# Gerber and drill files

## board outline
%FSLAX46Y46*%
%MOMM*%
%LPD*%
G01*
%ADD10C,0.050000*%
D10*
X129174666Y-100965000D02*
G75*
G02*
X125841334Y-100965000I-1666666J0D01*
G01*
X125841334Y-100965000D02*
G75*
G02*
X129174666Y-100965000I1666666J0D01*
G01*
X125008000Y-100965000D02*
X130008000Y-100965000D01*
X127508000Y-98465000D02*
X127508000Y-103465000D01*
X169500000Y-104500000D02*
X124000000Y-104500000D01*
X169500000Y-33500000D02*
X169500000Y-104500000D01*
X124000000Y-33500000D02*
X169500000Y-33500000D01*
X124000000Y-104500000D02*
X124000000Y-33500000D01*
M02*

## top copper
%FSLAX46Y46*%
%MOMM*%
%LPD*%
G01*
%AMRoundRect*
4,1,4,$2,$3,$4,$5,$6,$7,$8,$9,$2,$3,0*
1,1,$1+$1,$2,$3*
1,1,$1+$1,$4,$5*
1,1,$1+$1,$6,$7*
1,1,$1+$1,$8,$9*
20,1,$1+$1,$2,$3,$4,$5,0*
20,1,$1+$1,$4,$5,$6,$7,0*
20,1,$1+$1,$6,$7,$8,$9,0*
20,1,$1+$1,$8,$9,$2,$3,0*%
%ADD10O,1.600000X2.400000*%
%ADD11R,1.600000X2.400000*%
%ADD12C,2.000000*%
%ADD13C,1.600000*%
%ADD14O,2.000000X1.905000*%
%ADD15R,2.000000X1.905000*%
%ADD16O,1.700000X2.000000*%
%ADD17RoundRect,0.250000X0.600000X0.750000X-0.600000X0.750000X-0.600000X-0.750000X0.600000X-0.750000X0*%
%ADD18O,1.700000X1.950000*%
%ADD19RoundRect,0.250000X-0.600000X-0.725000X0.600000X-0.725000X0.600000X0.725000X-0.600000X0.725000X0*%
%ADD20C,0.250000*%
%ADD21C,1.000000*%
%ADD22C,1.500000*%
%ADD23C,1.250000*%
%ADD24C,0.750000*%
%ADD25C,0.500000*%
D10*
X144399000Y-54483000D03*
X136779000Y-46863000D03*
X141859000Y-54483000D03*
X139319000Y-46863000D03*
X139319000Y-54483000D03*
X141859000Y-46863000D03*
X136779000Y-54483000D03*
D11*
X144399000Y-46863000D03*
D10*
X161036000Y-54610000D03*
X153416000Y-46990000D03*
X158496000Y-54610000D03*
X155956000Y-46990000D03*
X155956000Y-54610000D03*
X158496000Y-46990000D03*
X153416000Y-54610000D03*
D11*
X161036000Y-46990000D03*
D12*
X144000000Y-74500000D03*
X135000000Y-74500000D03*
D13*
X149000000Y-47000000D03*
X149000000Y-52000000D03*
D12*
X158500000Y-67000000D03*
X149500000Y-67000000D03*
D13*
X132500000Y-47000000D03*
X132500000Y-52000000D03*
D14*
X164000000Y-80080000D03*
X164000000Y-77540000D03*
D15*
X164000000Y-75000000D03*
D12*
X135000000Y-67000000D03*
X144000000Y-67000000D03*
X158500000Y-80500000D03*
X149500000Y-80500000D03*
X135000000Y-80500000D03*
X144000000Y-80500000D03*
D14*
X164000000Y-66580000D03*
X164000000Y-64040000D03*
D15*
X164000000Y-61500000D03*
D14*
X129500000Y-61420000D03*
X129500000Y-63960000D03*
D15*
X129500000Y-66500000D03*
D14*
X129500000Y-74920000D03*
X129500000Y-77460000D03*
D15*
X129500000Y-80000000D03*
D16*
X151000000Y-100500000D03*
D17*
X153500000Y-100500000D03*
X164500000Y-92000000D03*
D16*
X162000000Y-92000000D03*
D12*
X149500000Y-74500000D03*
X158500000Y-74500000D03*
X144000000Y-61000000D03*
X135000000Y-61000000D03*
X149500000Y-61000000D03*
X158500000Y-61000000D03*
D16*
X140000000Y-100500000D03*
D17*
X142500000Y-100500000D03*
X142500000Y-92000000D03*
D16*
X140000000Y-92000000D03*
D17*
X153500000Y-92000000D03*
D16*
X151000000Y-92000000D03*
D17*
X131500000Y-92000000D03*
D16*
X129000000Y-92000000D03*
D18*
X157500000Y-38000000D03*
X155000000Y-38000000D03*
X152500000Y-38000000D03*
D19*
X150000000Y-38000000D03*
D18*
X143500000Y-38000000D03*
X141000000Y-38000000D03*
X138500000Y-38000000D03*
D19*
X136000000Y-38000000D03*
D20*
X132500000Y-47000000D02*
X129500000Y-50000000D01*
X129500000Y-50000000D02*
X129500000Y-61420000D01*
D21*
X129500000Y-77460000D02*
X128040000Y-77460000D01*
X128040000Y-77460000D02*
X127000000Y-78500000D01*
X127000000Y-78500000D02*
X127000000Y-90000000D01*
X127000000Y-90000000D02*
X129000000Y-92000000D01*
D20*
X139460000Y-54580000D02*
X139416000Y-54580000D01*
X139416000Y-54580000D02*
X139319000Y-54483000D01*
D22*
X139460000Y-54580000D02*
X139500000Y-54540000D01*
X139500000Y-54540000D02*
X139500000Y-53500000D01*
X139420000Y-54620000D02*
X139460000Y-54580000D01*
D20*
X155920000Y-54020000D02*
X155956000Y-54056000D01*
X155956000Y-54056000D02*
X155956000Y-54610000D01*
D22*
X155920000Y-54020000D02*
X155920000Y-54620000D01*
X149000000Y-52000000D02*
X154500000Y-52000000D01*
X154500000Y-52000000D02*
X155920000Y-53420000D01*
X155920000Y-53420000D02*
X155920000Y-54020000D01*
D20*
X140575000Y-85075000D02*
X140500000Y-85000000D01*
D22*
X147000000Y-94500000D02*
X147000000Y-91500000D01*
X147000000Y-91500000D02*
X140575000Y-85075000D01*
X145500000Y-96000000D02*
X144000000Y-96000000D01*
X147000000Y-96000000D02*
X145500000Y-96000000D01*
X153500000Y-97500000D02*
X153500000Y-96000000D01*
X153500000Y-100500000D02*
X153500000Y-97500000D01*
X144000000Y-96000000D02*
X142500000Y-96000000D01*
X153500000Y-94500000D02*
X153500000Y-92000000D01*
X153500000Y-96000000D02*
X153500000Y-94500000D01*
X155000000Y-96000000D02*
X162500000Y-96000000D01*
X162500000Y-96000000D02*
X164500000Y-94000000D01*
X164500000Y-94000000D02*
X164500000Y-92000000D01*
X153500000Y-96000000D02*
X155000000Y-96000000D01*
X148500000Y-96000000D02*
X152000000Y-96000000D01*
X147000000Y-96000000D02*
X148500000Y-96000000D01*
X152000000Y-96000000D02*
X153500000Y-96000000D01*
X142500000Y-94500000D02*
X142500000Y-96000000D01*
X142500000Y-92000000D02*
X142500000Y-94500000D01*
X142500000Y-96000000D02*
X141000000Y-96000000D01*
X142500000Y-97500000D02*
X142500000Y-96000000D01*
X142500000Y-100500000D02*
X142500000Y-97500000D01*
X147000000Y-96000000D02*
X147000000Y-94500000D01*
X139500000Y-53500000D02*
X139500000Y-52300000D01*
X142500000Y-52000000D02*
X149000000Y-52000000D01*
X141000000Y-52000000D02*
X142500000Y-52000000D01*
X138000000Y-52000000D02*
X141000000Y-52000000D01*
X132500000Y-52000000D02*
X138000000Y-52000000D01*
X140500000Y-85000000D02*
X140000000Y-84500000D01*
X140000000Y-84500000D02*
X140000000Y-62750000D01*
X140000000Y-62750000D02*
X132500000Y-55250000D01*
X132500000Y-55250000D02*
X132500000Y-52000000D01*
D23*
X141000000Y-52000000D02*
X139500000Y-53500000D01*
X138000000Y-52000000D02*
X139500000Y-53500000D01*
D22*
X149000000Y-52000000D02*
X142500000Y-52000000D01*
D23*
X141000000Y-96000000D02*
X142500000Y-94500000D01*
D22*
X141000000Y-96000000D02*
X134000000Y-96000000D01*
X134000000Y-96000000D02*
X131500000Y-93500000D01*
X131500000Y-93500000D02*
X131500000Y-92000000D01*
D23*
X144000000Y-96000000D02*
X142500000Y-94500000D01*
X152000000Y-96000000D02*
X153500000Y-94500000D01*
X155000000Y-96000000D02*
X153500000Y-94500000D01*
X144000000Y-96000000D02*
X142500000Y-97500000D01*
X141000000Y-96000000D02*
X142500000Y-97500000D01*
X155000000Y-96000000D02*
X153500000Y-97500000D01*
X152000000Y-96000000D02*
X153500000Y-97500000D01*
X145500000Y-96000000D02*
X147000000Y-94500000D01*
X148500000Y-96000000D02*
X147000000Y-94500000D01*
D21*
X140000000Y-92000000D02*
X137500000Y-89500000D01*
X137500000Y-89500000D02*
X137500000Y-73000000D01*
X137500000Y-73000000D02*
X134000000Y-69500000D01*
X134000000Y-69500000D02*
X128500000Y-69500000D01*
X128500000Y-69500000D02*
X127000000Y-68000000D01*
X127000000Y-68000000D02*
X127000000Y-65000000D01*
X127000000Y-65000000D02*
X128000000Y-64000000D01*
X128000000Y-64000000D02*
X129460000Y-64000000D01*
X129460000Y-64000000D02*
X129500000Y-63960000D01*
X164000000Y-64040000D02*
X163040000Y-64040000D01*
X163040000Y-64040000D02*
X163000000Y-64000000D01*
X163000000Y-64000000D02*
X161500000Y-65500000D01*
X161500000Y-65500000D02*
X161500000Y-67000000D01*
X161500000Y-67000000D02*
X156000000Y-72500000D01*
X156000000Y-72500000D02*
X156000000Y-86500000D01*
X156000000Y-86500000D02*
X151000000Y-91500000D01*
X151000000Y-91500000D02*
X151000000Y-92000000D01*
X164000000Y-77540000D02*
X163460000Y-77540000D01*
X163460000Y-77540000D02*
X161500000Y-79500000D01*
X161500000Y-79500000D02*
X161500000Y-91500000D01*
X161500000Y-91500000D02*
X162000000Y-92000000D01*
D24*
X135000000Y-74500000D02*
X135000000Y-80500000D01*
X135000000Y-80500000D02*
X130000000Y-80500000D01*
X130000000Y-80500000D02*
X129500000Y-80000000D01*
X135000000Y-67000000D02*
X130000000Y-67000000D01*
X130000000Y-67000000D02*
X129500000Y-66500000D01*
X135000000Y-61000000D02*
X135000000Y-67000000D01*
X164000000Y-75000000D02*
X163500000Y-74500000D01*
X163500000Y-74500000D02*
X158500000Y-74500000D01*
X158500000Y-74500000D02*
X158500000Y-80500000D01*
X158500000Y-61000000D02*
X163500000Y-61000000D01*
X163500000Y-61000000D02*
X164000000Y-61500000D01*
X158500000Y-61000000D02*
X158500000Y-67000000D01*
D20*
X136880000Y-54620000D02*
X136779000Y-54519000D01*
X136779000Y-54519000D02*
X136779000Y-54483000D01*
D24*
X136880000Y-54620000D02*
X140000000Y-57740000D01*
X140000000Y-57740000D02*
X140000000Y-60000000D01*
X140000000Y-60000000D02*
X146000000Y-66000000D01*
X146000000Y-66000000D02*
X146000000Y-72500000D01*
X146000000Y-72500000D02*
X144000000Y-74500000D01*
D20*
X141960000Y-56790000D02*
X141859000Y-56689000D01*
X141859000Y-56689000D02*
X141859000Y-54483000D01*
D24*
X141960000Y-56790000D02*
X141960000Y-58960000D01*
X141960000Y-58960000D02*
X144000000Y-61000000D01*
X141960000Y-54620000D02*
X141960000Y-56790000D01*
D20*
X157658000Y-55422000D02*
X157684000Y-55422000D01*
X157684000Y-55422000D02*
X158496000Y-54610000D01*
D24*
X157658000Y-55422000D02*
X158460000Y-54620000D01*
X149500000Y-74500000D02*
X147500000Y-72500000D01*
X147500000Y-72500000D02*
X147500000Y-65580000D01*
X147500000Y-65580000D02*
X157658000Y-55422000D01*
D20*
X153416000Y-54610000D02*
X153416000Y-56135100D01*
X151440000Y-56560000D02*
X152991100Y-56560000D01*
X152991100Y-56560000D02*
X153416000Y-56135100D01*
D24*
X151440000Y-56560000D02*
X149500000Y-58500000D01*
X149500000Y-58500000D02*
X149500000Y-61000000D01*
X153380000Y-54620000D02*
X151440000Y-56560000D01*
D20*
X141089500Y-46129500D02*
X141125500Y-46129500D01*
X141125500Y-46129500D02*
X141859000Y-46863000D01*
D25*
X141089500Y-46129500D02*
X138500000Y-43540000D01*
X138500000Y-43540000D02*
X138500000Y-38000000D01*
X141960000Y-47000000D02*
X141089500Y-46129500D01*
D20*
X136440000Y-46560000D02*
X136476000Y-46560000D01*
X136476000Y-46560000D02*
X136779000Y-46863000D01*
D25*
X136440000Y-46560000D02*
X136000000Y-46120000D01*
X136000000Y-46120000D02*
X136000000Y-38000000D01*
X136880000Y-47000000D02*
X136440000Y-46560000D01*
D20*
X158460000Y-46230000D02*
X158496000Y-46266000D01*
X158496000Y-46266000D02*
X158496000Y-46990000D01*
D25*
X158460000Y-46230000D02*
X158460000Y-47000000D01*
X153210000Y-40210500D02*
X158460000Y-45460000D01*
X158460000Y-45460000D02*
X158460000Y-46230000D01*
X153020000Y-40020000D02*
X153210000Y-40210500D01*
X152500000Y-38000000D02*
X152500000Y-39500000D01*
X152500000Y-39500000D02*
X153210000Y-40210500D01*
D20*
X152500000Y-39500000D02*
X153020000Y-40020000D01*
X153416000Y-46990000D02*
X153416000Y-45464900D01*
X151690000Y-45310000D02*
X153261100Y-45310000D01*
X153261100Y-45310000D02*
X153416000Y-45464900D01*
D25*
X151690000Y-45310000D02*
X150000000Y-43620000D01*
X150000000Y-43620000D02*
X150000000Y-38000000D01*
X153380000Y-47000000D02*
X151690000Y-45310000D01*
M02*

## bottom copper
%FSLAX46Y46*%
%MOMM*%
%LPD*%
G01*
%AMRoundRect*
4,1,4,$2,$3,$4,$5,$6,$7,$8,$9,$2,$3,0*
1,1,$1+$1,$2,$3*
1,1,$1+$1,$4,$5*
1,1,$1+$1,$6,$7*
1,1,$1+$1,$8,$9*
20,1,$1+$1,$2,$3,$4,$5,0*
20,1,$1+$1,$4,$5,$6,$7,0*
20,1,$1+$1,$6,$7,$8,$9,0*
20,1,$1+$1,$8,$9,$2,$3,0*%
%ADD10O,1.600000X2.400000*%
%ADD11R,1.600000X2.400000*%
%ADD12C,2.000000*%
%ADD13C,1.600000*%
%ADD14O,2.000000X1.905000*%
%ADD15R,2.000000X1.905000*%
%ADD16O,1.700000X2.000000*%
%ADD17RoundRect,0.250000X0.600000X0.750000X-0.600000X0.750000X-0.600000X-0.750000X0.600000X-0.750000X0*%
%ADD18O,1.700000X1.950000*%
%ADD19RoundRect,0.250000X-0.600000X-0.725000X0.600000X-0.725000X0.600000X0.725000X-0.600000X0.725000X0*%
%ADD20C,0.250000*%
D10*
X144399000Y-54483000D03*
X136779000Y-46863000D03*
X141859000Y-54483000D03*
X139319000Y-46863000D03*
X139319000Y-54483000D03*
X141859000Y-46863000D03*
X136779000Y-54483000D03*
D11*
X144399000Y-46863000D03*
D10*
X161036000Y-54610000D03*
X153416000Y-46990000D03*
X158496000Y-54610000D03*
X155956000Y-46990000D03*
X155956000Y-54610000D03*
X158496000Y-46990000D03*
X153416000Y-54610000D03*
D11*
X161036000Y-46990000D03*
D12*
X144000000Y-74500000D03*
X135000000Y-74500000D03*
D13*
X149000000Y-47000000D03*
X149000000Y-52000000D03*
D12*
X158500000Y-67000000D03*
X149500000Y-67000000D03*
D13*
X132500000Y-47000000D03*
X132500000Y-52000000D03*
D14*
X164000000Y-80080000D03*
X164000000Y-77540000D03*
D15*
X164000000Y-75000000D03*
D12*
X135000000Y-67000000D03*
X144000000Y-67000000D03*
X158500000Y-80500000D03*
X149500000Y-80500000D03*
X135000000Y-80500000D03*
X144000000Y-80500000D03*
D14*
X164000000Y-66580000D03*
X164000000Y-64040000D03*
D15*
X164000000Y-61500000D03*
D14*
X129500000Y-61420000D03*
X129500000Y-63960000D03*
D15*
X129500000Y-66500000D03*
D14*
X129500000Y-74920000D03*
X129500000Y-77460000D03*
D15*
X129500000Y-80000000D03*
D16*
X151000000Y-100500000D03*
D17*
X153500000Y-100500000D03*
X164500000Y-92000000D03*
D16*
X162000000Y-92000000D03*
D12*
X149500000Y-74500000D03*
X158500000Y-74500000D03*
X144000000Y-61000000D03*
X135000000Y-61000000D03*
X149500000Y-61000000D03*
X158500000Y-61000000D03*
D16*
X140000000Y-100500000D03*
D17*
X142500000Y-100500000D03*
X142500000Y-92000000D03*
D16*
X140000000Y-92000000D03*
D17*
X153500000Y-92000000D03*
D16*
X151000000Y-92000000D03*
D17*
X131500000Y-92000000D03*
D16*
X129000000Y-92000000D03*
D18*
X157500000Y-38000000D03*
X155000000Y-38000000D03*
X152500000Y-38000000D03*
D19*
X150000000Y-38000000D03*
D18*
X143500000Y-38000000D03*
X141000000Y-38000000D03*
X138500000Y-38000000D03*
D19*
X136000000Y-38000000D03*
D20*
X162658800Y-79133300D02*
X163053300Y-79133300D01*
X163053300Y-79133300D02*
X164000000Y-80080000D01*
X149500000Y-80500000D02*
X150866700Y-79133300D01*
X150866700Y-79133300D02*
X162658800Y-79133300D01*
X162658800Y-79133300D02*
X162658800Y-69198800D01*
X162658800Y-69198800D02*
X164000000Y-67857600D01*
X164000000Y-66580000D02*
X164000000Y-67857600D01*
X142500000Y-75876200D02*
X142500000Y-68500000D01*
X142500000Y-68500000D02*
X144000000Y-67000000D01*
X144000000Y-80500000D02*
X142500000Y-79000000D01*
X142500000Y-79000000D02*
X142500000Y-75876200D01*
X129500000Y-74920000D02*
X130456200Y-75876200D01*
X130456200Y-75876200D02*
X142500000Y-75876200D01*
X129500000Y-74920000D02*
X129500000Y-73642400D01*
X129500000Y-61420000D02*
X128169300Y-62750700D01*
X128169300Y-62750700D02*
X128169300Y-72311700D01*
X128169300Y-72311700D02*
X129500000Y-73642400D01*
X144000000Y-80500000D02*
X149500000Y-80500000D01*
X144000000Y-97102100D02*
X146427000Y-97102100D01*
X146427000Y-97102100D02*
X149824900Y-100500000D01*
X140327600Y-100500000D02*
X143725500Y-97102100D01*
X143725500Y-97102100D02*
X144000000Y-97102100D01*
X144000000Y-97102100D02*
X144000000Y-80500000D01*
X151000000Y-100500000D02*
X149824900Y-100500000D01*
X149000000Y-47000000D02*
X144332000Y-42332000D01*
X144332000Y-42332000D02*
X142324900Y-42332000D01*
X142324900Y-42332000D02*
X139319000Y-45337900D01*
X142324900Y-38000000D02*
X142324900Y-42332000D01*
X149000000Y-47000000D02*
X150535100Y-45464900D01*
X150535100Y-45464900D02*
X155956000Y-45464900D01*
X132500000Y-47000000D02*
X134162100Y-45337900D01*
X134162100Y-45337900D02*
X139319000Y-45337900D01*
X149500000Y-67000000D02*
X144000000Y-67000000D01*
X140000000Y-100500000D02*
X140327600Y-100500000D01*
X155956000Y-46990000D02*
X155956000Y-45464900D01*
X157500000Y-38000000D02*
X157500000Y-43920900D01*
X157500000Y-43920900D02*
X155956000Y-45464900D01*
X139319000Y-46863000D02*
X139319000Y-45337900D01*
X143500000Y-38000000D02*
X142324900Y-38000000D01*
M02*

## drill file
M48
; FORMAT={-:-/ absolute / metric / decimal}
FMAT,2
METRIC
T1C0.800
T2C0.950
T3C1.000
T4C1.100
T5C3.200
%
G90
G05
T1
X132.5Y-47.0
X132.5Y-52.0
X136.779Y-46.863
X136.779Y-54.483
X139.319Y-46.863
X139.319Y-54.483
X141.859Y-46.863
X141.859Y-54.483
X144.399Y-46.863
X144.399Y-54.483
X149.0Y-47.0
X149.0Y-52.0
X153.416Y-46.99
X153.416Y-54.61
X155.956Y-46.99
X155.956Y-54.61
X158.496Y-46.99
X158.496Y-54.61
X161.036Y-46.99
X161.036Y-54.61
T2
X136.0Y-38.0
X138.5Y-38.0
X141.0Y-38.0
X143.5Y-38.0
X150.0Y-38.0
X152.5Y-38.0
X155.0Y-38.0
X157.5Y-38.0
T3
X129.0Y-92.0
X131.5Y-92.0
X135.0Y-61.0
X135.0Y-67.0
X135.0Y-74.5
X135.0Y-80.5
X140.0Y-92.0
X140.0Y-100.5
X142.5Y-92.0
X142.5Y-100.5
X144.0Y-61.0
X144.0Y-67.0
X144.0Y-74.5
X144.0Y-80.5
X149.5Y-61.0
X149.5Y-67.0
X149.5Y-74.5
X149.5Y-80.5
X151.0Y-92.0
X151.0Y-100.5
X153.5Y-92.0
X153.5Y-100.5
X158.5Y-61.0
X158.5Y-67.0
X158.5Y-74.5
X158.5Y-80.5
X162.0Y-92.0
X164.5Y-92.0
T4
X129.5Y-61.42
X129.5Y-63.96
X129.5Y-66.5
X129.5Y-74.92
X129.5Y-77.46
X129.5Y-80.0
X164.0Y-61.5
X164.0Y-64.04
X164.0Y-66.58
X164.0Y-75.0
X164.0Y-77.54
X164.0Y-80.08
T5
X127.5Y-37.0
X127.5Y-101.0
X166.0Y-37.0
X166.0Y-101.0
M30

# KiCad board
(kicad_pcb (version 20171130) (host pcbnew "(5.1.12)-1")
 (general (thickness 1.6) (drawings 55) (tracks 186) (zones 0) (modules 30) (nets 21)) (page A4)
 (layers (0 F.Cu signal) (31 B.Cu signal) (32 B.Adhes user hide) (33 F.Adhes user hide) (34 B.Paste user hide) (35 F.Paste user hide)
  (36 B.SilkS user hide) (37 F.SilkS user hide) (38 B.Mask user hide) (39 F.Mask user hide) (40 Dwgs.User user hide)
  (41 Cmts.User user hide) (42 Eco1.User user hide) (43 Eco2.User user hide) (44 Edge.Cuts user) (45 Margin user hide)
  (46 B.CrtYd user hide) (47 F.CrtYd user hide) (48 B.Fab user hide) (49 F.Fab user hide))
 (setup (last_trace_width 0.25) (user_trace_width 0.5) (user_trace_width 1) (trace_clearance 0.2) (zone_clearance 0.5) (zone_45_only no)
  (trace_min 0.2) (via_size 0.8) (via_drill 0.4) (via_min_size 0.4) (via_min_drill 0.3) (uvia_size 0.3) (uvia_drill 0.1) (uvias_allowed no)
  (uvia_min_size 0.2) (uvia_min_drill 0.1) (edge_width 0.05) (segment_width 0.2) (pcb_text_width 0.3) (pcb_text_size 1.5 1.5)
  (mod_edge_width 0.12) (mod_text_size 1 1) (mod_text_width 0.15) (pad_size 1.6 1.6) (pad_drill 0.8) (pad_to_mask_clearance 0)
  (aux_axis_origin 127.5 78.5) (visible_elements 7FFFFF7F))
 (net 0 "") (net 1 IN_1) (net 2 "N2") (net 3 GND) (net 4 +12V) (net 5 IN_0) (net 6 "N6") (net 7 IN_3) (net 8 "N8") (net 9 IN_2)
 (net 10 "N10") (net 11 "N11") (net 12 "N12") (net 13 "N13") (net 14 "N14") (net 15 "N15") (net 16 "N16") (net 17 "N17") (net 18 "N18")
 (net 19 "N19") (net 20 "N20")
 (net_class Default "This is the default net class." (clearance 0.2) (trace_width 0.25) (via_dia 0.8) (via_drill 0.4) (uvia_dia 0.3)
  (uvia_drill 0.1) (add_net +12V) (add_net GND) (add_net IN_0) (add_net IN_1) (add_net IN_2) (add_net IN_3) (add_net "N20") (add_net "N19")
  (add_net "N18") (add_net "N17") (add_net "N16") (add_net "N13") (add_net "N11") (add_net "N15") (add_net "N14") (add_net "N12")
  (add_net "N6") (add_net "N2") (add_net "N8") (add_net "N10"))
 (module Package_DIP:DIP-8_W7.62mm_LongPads (layer F.Cu) (at 144.399 46.863 270)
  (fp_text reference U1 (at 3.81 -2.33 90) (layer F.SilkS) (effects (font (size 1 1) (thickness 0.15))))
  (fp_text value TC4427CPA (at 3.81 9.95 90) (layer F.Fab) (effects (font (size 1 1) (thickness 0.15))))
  (pad 8 thru_hole oval (at 7.62 0 270) (size 2.4 1.6) (drill 0.8) (layers *.Cu *.Mask))
  (pad 4 thru_hole oval (at 0 7.62 270) (size 2.4 1.6) (drill 0.8) (layers *.Cu *.Mask) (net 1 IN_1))
  (pad 7 thru_hole oval (at 7.62 2.54 270) (size 2.4 1.6) (drill 0.8) (layers *.Cu *.Mask) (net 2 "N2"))
  (pad 3 thru_hole oval (at 0 5.08 270) (size 2.4 1.6) (drill 0.8) (layers *.Cu *.Mask) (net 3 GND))
  (pad 6 thru_hole oval (at 7.62 5.08 270) (size 2.4 1.6) (drill 0.8) (layers *.Cu *.Mask) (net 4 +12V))
  (pad 2 thru_hole oval (at 0 2.54 270) (size 2.4 1.6) (drill 0.8) (layers *.Cu *.Mask) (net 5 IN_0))
  (pad 5 thru_hole oval (at 7.62 7.62 270) (size 2.4 1.6) (drill 0.8) (layers *.Cu *.Mask) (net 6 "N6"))
  (pad 1 thru_hole rect (at 0 0 270) (size 2.4 1.6) (drill 0.8) (layers *.Cu *.Mask)))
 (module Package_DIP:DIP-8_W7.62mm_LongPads (layer F.Cu) (at 161.036 46.99 270)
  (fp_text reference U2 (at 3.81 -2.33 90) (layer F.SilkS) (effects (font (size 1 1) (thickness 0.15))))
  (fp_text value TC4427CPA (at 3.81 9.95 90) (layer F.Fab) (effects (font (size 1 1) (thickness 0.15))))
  (pad 8 thru_hole oval (at 7.62 0 270) (size 2.4 1.6) (drill 0.8) (layers *.Cu *.Mask))
  (pad 4 thru_hole oval (at 0 7.62 270) (size 2.4 1.6) (drill 0.8) (layers *.Cu *.Mask) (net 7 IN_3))
  (pad 7 thru_hole oval (at 7.62 2.54 270) (size 2.4 1.6) (drill 0.8) (layers *.Cu *.Mask) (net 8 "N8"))
  (pad 3 thru_hole oval (at 0 5.08 270) (size 2.4 1.6) (drill 0.8) (layers *.Cu *.Mask) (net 3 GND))
  (pad 6 thru_hole oval (at 7.62 5.08 270) (size 2.4 1.6) (drill 0.8) (layers *.Cu *.Mask) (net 4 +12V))
  (pad 2 thru_hole oval (at 0 2.54 270) (size 2.4 1.6) (drill 0.8) (layers *.Cu *.Mask) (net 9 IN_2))
  (pad 5 thru_hole oval (at 7.62 7.62 270) (size 2.4 1.6) (drill 0.8) (layers *.Cu *.Mask) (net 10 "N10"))
  (pad 1 thru_hole rect (at 0 0 270) (size 2.4 1.6) (drill 0.8) (layers *.Cu *.Mask)))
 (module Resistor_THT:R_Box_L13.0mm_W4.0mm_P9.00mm (layer F.Cu) (at 144 74.5 180)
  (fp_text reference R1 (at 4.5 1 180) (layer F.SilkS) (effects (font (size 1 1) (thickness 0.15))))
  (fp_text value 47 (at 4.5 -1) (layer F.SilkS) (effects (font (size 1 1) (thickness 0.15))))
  (pad 1 thru_hole circle (at 0 0 180) (size 2 2) (drill 1) (layers *.Cu *.Mask) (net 6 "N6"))
  (pad 2 thru_hole circle (at 9 0 180) (size 2 2) (drill 1) (layers *.Cu *.Mask) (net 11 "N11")))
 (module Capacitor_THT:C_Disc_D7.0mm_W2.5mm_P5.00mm (layer F.Cu) (at 149 52 90)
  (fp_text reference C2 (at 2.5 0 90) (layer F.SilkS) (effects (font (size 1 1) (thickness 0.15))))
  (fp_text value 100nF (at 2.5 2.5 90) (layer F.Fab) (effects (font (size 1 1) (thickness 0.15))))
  (pad 2 thru_hole circle (at 5 0 90) (size 1.6 1.6) (drill 0.8) (layers *.Cu *.Mask) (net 3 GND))
  (pad 1 thru_hole circle (at 0 0 90) (size 1.6 1.6) (drill 0.8) (layers *.Cu *.Mask) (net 4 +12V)))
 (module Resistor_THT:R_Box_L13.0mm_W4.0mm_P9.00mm (layer F.Cu) (at 149.5 67)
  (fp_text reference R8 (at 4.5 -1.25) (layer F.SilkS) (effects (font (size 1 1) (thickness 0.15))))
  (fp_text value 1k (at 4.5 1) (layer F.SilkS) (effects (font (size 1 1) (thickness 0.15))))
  (pad 2 thru_hole circle (at 9 0) (size 2 2) (drill 1) (layers *.Cu *.Mask) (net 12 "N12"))
  (pad 1 thru_hole circle (at 0 0) (size 2 2) (drill 1) (layers *.Cu *.Mask) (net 3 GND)))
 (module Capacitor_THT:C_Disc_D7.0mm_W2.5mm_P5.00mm (layer F.Cu) (at 132.5 52 90)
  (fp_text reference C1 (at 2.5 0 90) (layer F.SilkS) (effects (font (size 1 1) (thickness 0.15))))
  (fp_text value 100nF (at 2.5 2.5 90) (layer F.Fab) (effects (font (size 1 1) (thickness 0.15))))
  (pad 2 thru_hole circle (at 5 0 90) (size 1.6 1.6) (drill 0.8) (layers *.Cu *.Mask) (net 3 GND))
  (pad 1 thru_hole circle (at 0 0 90) (size 1.6 1.6) (drill 0.8) (layers *.Cu *.Mask) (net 4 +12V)))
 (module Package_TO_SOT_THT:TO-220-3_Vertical (layer F.Cu) (at 164 75 270)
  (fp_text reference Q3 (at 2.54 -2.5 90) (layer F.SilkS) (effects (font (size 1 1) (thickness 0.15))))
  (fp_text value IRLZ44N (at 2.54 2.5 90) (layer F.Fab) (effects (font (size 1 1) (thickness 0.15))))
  (pad 3 thru_hole oval (at 5.08 0 270) (size 1.905 2) (drill 1.1) (layers *.Cu *.Mask) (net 3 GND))
  (pad 2 thru_hole oval (at 2.54 0 270) (size 1.905 2) (drill 1.1) (layers *.Cu *.Mask) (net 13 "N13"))
  (pad 1 thru_hole rect (at 0 0 270) (size 1.905 2) (drill 1.1) (layers *.Cu *.Mask) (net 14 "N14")))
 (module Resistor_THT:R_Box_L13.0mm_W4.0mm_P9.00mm (layer F.Cu) (at 144 67 180)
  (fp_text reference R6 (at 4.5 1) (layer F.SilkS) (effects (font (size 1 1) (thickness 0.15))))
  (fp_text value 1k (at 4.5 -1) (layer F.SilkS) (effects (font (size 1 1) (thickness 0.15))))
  (pad 2 thru_hole circle (at 9 0 180) (size 2 2) (drill 1) (layers *.Cu *.Mask) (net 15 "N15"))
  (pad 1 thru_hole circle (at 0 0 180) (size 2 2) (drill 1) (layers *.Cu *.Mask) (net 3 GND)))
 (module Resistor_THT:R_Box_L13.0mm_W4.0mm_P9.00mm (layer F.Cu) (at 149.5 80.5)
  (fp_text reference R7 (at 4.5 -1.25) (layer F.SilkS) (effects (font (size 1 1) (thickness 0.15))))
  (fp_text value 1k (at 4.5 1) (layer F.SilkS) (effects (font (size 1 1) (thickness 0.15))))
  (pad 2 thru_hole circle (at 9 0) (size 2 2) (drill 1) (layers *.Cu *.Mask) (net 14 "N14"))
  (pad 1 thru_hole circle (at 0 0) (size 2 2) (drill 1) (layers *.Cu *.Mask) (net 3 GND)))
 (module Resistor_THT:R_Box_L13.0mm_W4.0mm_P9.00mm (layer F.Cu) (at 144 80.5 180)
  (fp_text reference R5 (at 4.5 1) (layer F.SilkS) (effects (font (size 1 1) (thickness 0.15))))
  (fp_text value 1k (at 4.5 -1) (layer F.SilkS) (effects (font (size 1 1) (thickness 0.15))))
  (pad 2 thru_hole circle (at 9 0 180) (size 2 2) (drill 1) (layers *.Cu *.Mask) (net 11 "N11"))
  (pad 1 thru_hole circle (at 0 0 180) (size 2 2) (drill 1) (layers *.Cu *.Mask) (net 3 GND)))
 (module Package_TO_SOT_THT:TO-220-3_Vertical (layer F.Cu) (at 164 61.5 270)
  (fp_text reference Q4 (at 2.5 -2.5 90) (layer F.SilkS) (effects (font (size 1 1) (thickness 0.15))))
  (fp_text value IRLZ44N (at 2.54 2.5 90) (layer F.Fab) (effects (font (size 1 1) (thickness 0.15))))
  (pad 3 thru_hole oval (at 5.08 0 270) (size 1.905 2) (drill 1.1) (layers *.Cu *.Mask) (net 3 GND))
  (pad 2 thru_hole oval (at 2.54 0 270) (size 1.905 2) (drill 1.1) (layers *.Cu *.Mask) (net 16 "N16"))
  (pad 1 thru_hole rect (at 0 0 270) (size 1.905 2) (drill 1.1) (layers *.Cu *.Mask) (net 12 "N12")))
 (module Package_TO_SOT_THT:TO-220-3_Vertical (layer F.Cu) (at 129.5 66.5 90)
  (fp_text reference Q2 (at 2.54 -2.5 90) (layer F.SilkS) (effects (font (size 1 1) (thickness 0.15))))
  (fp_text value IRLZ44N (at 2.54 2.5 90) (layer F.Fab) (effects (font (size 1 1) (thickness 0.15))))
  (pad 3 thru_hole oval (at 5.08 0 90) (size 1.905 2) (drill 1.1) (layers *.Cu *.Mask) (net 3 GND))
  (pad 2 thru_hole oval (at 2.54 0 90) (size 1.905 2) (drill 1.1) (layers *.Cu *.Mask) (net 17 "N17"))
  (pad 1 thru_hole rect (at 0 0 90) (size 1.905 2) (drill 1.1) (layers *.Cu *.Mask) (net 15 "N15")))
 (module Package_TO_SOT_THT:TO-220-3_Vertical (layer F.Cu) (at 129.5 80 90)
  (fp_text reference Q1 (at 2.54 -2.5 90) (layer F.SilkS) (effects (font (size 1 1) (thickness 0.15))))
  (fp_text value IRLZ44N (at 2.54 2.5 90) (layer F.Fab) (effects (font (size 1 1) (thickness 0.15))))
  (pad 3 thru_hole oval (at 5.08 0 90) (size 1.905 2) (drill 1.1) (layers *.Cu *.Mask) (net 3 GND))
  (pad 2 thru_hole oval (at 2.54 0 90) (size 1.905 2) (drill 1.1) (layers *.Cu *.Mask) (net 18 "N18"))
  (pad 1 thru_hole rect (at 0 0 90) (size 1.905 2) (drill 1.1) (layers *.Cu *.Mask) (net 11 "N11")))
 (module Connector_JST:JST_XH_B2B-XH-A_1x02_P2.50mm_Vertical (layer F.Cu) (at 153.5 100.5 180)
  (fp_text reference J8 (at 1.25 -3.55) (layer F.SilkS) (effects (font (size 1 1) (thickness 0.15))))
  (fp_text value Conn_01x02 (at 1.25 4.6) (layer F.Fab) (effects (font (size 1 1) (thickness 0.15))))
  (pad 2 thru_hole oval (at 2.5 0 180) (size 1.7 2) (drill 1) (layers *.Cu *.Mask) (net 3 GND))
  (pad 1 thru_hole roundrect (at 0 0 180) (size 1.7 2) (drill 1) (layers *.Cu *.Mask) (roundrect_rratio 0.1470588235294118) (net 4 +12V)))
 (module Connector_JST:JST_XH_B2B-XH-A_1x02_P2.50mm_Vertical (layer F.Cu) (at 164.5 92 180)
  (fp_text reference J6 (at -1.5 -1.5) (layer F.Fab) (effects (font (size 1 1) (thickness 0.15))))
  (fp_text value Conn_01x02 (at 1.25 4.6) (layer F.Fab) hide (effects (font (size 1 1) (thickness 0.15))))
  (pad 1 thru_hole roundrect (at 0 0 180) (size 1.7 2) (drill 1) (layers *.Cu *.Mask) (roundrect_rratio 0.1470588235294118) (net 4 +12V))
  (pad 2 thru_hole oval (at 2.5 0 180) (size 1.7 2) (drill 1) (layers *.Cu *.Mask) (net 13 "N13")))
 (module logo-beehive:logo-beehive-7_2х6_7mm (layer F.Cu) (at 133 99.5 90)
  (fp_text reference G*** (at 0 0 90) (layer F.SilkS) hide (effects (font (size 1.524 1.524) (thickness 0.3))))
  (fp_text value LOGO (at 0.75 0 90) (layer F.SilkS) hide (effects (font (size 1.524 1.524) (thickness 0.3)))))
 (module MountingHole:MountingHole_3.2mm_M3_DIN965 (layer F.Cu) (at 166 37 270)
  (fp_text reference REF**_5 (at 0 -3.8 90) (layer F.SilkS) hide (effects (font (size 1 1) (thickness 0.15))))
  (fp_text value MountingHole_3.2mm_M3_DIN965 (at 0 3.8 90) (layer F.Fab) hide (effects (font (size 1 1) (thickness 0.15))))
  (pad 1 np_thru_hole circle (at 0 0 270) (size 3.2 3.2) (drill 3.2) (layers *.Cu *.Mask)))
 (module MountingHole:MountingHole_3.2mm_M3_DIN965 (layer F.Cu) (at 166 101 180)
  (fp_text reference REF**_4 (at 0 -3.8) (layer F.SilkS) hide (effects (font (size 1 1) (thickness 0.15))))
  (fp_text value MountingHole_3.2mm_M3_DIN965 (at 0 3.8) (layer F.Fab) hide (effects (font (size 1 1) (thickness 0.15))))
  (pad 1 np_thru_hole circle (at 0 0 180) (size 3.2 3.2) (drill 3.2) (layers *.Cu *.Mask)))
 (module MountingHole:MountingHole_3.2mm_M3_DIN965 (layer F.Cu) (at 127.5 101 90)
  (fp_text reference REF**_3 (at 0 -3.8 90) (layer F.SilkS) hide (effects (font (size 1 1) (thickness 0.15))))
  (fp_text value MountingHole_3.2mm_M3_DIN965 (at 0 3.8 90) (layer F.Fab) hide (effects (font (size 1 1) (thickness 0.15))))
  (pad 1 np_thru_hole circle (at 0 0 90) (size 3.2 3.2) (drill 3.2) (layers *.Cu *.Mask)))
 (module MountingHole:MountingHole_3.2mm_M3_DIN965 (layer F.Cu) (at 127.5 37 90)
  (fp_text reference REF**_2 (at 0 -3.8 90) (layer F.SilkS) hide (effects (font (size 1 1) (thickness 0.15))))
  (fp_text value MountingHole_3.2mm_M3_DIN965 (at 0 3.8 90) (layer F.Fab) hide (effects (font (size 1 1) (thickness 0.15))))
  (pad 1 np_thru_hole circle (at 0 0 90) (size 3.2 3.2) (drill 3.2) (layers *.Cu *.Mask)))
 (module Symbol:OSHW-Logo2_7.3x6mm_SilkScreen (layer F.Cu) (at 128.5 55)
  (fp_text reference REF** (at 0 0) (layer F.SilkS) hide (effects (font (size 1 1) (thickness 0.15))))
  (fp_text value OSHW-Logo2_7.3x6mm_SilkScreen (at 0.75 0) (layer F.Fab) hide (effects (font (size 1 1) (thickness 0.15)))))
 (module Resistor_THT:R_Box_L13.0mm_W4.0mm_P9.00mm (layer F.Cu) (at 149.5 74.5)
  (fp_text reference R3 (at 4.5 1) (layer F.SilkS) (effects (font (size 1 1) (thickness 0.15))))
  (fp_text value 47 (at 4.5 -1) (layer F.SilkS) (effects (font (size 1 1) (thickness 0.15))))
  (pad 1 thru_hole circle (at 0 0) (size 2 2) (drill 1) (layers *.Cu *.Mask) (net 8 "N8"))
  (pad 2 thru_hole circle (at 9 0) (size 2 2) (drill 1) (layers *.Cu *.Mask) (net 14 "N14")))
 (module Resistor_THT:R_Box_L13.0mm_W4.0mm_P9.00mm (layer F.Cu) (at 144 61 180)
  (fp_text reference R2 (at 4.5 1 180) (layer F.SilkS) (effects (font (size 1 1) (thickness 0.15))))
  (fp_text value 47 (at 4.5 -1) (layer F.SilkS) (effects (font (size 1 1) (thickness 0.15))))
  (pad 1 thru_hole circle (at 0 0 180) (size 2 2) (drill 1) (layers *.Cu *.Mask) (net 2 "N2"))
  (pad 2 thru_hole circle (at 9 0 180) (size 2 2) (drill 1) (layers *.Cu *.Mask) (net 15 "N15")))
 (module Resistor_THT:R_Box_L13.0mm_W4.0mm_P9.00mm (layer F.Cu) (at 149.5 61)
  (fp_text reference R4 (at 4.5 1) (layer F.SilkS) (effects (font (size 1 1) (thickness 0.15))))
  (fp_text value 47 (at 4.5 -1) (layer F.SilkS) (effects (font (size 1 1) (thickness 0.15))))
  (pad 1 thru_hole circle (at 0 0) (size 2 2) (drill 1) (layers *.Cu *.Mask) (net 10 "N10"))
  (pad 2 thru_hole circle (at 9 0) (size 2 2) (drill 1) (layers *.Cu *.Mask) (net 12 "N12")))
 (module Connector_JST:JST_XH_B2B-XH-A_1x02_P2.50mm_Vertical (layer F.Cu) (at 142.5 100.5 180)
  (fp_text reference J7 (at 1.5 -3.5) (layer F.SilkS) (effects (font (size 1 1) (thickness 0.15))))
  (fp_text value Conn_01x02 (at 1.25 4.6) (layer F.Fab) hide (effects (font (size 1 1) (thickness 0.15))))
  (pad 2 thru_hole oval (at 2.5 0 180) (size 1.7 2) (drill 1) (layers *.Cu *.Mask) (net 3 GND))
  (pad 1 thru_hole roundrect (at 0 0 180) (size 1.7 2) (drill 1) (layers *.Cu *.Mask) (roundrect_rratio 0.1470588235294118) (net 4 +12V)))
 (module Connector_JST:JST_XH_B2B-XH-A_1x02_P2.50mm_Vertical (layer F.Cu) (at 142.5 92 180)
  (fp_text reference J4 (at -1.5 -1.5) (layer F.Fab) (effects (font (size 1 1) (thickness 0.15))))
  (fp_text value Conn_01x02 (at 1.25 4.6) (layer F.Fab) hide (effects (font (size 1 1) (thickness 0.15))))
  (pad 1 thru_hole roundrect (at 0 0 180) (size 1.7 2) (drill 1) (layers *.Cu *.Mask) (roundrect_rratio 0.1470588235294118) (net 4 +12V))
  (pad 2 thru_hole oval (at 2.5 0 180) (size 1.7 2) (drill 1) (layers *.Cu *.Mask) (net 17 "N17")))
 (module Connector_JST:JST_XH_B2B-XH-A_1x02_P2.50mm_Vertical (layer F.Cu) (at 153.5 92 180)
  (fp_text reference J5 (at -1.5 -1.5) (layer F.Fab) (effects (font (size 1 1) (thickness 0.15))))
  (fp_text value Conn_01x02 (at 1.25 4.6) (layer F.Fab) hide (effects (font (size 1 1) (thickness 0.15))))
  (pad 1 thru_hole roundrect (at 0 0 180) (size 1.7 2) (drill 1) (layers *.Cu *.Mask) (roundrect_rratio 0.1470588235294118) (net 4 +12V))
  (pad 2 thru_hole oval (at 2.5 0 180) (size 1.7 2) (drill 1) (layers *.Cu *.Mask) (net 16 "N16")))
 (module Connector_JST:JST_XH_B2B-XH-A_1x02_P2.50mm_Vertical (layer F.Cu) (at 131.5 92 180)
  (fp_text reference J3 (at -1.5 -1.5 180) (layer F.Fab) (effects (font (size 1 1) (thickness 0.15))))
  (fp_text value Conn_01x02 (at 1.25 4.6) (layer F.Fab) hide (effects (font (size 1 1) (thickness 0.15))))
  (pad 1 thru_hole roundrect (at 0 0 180) (size 1.7 2) (drill 1) (layers *.Cu *.Mask) (roundrect_rratio 0.1470588235294118) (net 4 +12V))
  (pad 2 thru_hole oval (at 2.5 0 180) (size 1.7 2) (drill 1) (layers *.Cu *.Mask) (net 18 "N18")))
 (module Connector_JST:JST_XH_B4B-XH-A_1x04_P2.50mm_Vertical (layer F.Cu) (at 150 38)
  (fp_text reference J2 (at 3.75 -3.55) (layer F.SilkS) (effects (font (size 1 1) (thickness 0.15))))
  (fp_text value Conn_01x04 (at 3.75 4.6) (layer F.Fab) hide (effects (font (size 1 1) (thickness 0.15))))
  (pad 4 thru_hole oval (at 7.5 0) (size 1.7 1.95) (drill 0.95) (layers *.Cu *.Mask) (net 3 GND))
  (pad 3 thru_hole oval (at 5 0) (size 1.7 1.95) (drill 0.95) (layers *.Cu *.Mask) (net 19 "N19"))
  (pad 2 thru_hole oval (at 2.5 0) (size 1.7 1.95) (drill 0.95) (layers *.Cu *.Mask) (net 9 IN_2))
  (pad 1 thru_hole roundrect (at 0 0) (size 1.7 1.95) (drill 0.95) (layers *.Cu *.Mask) (roundrect_rratio 0.1470588235294118) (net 7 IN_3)))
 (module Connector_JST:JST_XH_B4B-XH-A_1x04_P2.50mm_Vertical (layer F.Cu) (at 136 38)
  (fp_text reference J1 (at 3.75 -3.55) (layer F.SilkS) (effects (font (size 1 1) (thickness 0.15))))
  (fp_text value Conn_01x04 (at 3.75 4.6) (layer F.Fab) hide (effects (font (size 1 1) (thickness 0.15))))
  (pad 4 thru_hole oval (at 7.5 0) (size 1.7 1.95) (drill 0.95) (layers *.Cu *.Mask) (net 3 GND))
  (pad 3 thru_hole oval (at 5 0) (size 1.7 1.95) (drill 0.95) (layers *.Cu *.Mask) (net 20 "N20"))
  (pad 2 thru_hole oval (at 2.5 0) (size 1.7 1.95) (drill 0.95) (layers *.Cu *.Mask) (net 5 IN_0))
  (pad 1 thru_hole roundrect (at 0 0) (size 1.7 1.95) (drill 0.95) (layers *.Cu *.Mask) (roundrect_rratio 0.1470588235294118) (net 1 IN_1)))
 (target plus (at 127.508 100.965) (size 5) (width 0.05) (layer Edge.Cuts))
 (gr_line (start 169.5 104.5) (end 124 104.5) (layer Edge.Cuts) (width 0.05))
 (gr_line (start 169.5 33.5) (end 169.5 104.5) (layer Edge.Cuts) (width 0.05))
 (gr_line (start 124 33.5) (end 169.5 33.5) (layer Edge.Cuts) (width 0.05))
 (gr_line (start 124 104.5) (end 124 33.5) (layer Edge.Cuts) (width 0.05))
 (segment (start 162.6588 79.1333) (end 163.0533 79.1333) (width 0.25) (layer B.Cu) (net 3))
 (segment (start 163.0533 79.1333) (end 164 80.08) (width 0.25) (layer B.Cu) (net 3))
 (segment (start 149.5 80.5) (end 150.8667 79.1333) (width 0.25) (layer B.Cu) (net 3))
 (segment (start 150.8667 79.1333) (end 162.6588 79.1333) (width 0.25) (layer B.Cu) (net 3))
 (segment (start 162.6588 79.1333) (end 162.6588 69.1988) (width 0.25) (layer B.Cu) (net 3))
 (segment (start 162.6588 69.1988) (end 164 67.8576) (width 0.25) (layer B.Cu) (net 3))
 (segment (start 164 66.58) (end 164 67.8576) (width 0.25) (layer B.Cu) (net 3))
 (segment (start 142.5 75.8762) (end 142.5 68.5) (width 0.25) (layer B.Cu) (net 3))
 (segment (start 142.5 68.5) (end 144 67) (width 0.25) (layer B.Cu) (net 3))
 (segment (start 144 80.5) (end 142.5 79) (width 0.25) (layer B.Cu) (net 3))
 (segment (start 142.5 79) (end 142.5 75.8762) (width 0.25) (layer B.Cu) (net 3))
 (segment (start 129.5 74.92) (end 130.4562 75.8762) (width 0.25) (layer B.Cu) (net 3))
 (segment (start 130.4562 75.8762) (end 142.5 75.8762) (width 0.25) (layer B.Cu) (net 3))
 (segment (start 129.5 74.92) (end 129.5 73.6424) (width 0.25) (layer B.Cu) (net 3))
 (segment (start 129.5 61.42) (end 128.1693 62.7507) (width 0.25) (layer B.Cu) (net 3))
 (segment (start 128.1693 62.7507) (end 128.1693 72.3117) (width 0.25) (layer B.Cu) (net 3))
 (segment (start 128.1693 72.3117) (end 129.5 73.6424) (width 0.25) (layer B.Cu) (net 3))
 (segment (start 132.5 47) (end 129.5 50) (width 0.25) (layer F.Cu) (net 3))
 (segment (start 129.5 50) (end 129.5 61.42) (width 0.25) (layer F.Cu) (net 3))
 (segment (start 144 80.5) (end 149.5 80.5) (width 0.25) (layer B.Cu) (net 3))
 (segment (start 144 97.1021) (end 146.427 97.1021) (width 0.25) (layer B.Cu) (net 3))
 (segment (start 146.427 97.1021) (end 149.8249 100.5) (width 0.25) (layer B.Cu) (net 3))
 (segment (start 140.3276 100.5) (end 143.7255 97.1021) (width 0.25) (layer B.Cu) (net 3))
 (segment (start 143.7255 97.1021) (end 144 97.1021) (width 0.25) (layer B.Cu) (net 3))
 (segment (start 144 97.1021) (end 144 80.5) (width 0.25) (layer B.Cu) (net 3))
 (segment (start 151 100.5) (end 149.8249 100.5) (width 0.25) (layer B.Cu) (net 3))
 (segment (start 149 47) (end 144.332 42.332) (width 0.25) (layer B.Cu) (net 3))
 (segment (start 144.332 42.332) (end 142.3249 42.332) (width 0.25) (layer B.Cu) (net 3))
 (segment (start 142.3249 42.332) (end 139.319 45.3379) (width 0.25) (layer B.Cu) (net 3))
 (segment (start 142.3249 38) (end 142.3249 42.332) (width 0.25) (layer B.Cu) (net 3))
 (segment (start 149 47) (end 150.5351 45.4649) (width 0.25) (layer B.Cu) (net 3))
 (segment (start 150.5351 45.4649) (end 155.956 45.4649) (width 0.25) (layer B.Cu) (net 3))
 (segment (start 132.5 47) (end 134.1621 45.3379) (width 0.25) (layer B.Cu) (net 3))
 (segment (start 134.1621 45.3379) (end 139.319 45.3379) (width 0.25) (layer B.Cu) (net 3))
 (segment (start 149.5 67) (end 144 67) (width 0.25) (layer B.Cu) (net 3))
 (segment (start 140 100.5) (end 140.3276 100.5) (width 0.25) (layer B.Cu) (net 3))
 (segment (start 155.956 46.99) (end 155.956 45.4649) (width 0.25) (layer B.Cu) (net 3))
 (segment (start 157.5 38) (end 157.5 43.9209) (width 0.25) (layer B.Cu) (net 3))
 (segment (start 157.5 43.9209) (end 155.956 45.4649) (width 0.25) (layer B.Cu) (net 3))
 (segment (start 139.319 46.863) (end 139.319 45.3379) (width 0.25) (layer B.Cu) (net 3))
 (segment (start 143.5 38) (end 142.3249 38) (width 0.25) (layer B.Cu) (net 3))
 (segment (start 129.5 77.46) (end 128.04 77.46) (width 1) (layer F.Cu) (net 18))
 (segment (start 128.04 77.46) (end 127 78.5) (width 1) (layer F.Cu) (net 18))
 (segment (start 127 78.5) (end 127 90) (width 1) (layer F.Cu) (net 18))
 (segment (start 127 90) (end 129 92) (width 1) (layer F.Cu) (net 18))
 (segment (start 139.46 54.58) (end 139.416 54.58) (width 0.25) (layer F.Cu) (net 4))
 (segment (start 139.416 54.58) (end 139.319 54.483) (width 0.25) (layer F.Cu) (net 4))
 (segment (start 139.46 54.58) (end 139.5 54.54) (width 1.5) (layer F.Cu) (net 4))
 (segment (start 139.5 54.54) (end 139.5 53.5) (width 1.5) (layer F.Cu) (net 4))
 (segment (start 139.42 54.62) (end 139.46 54.58) (width 1.5) (layer F.Cu) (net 4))
 (segment (start 155.92 54.02) (end 155.956 54.056) (width 0.25) (layer F.Cu) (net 4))
 (segment (start 155.956 54.056) (end 155.956 54.61) (width 0.25) (layer F.Cu) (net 4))
 (segment (start 155.92 54.02) (end 155.92 54.62) (width 1.5) (layer F.Cu) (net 4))
 (segment (start 149 52) (end 154.5 52) (width 1.5) (layer F.Cu) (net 4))
 (segment (start 154.5 52) (end 155.92 53.42) (width 1.5) (layer F.Cu) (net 4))
 (segment (start 155.92 53.42) (end 155.92 54.02) (width 1.5) (layer F.Cu) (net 4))
 (segment (start 140.575 85.075) (end 140.5 85) (width 0.25) (layer F.Cu) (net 4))
 (segment (start 147 94.5) (end 147 91.5) (width 1.5) (layer F.Cu) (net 4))
 (segment (start 147 91.5) (end 140.575 85.075) (width 1.5) (layer F.Cu) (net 4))
 (segment (start 145.5 96) (end 144 96) (width 1.5) (layer F.Cu) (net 4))
 (segment (start 147 96) (end 145.5 96) (width 1.5) (layer F.Cu) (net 4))
 (segment (start 153.5 97.5) (end 153.5 96) (width 1.5) (layer F.Cu) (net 4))
 (segment (start 153.5 100.5) (end 153.5 97.5) (width 1.5) (layer F.Cu) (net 4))
 (segment (start 144 96) (end 142.5 96) (width 1.5) (layer F.Cu) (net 4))
 (segment (start 153.5 94.5) (end 153.5 92) (width 1.5) (layer F.Cu) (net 4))
 (segment (start 153.5 96) (end 153.5 94.5) (width 1.5) (layer F.Cu) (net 4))
 (segment (start 155 96) (end 162.5 96) (width 1.5) (layer F.Cu) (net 4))
 (segment (start 162.5 96) (end 164.5 94) (width 1.5) (layer F.Cu) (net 4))
 (segment (start 164.5 94) (end 164.5 92) (width 1.5) (layer F.Cu) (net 4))
 (segment (start 153.5 96) (end 155 96) (width 1.5) (layer F.Cu) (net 4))
 (segment (start 148.5 96) (end 152 96) (width 1.5) (layer F.Cu) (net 4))
 (segment (start 147 96) (end 148.5 96) (width 1.5) (layer F.Cu) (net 4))
 (segment (start 152 96) (end 153.5 96) (width 1.5) (layer F.Cu) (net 4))
 (segment (start 142.5 94.5) (end 142.5 96) (width 1.5) (layer F.Cu) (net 4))
 (segment (start 142.5 92) (end 142.5 94.5) (width 1.5) (layer F.Cu) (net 4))
 (segment (start 142.5 96) (end 141 96) (width 1.5) (layer F.Cu) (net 4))
 (segment (start 142.5 97.5) (end 142.5 96) (width 1.5) (layer F.Cu) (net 4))
 (segment (start 142.5 100.5) (end 142.5 97.5) (width 1.5) (layer F.Cu) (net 4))
 (segment (start 147 96) (end 147 94.5) (width 1.5) (layer F.Cu) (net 4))
 (segment (start 139.5 53.5) (end 139.5 52.3) (width 1.5) (layer F.Cu) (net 4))
 (segment (start 142.5 52) (end 149 52) (width 1.5) (layer F.Cu) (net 4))
 (segment (start 141 52) (end 142.5 52) (width 1.5) (layer F.Cu) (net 4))
 (segment (start 138 52) (end 141 52) (width 1.5) (layer F.Cu) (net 4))
 (segment (start 132.5 52) (end 138 52) (width 1.5) (layer F.Cu) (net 4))
 (segment (start 140.5 85) (end 140 84.5) (width 1.5) (layer F.Cu) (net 4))
 (segment (start 140 84.5) (end 140 62.75) (width 1.5) (layer F.Cu) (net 4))
 (segment (start 140 62.75) (end 132.5 55.25) (width 1.5) (layer F.Cu) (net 4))
 (segment (start 132.5 55.25) (end 132.5 52) (width 1.5) (layer F.Cu) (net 4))
 (segment (start 141 52) (end 139.5 53.5) (width 1.25) (layer F.Cu) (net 4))
 (segment (start 138 52) (end 139.5 53.5) (width 1.25) (layer F.Cu) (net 4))
 (segment (start 149 52) (end 142.5 52) (width 1.5) (layer F.Cu) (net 4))
 (segment (start 141 96) (end 142.5 94.5) (width 1.25) (layer F.Cu) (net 4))
 (segment (start 141 96) (end 134 96) (width 1.5) (layer F.Cu) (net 4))
 (segment (start 134 96) (end 131.5 93.5) (width 1.5) (layer F.Cu) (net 4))
 (segment (start 131.5 93.5) (end 131.5 92) (width 1.5) (layer F.Cu) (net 4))
 (segment (start 144 96) (end 142.5 94.5) (width 1.25) (layer F.Cu) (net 4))
 (segment (start 152 96) (end 153.5 94.5) (width 1.25) (layer F.Cu) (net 4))
 (segment (start 155 96) (end 153.5 94.5) (width 1.25) (layer F.Cu) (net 4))
 (segment (start 144 96) (end 142.5 97.5) (width 1.25) (layer F.Cu) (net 4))
 (segment (start 141 96) (end 142.5 97.5) (width 1.25) (layer F.Cu) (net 4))
 (segment (start 155 96) (end 153.5 97.5) (width 1.25) (layer F.Cu) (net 4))
 (segment (start 152 96) (end 153.5 97.5) (width 1.25) (layer F.Cu) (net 4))
 (segment (start 145.5 96) (end 147 94.5) (width 1.25) (layer F.Cu) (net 4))
 (segment (start 148.5 96) (end 147 94.5) (width 1.25) (layer F.Cu) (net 4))
 (segment (start 140 92) (end 137.5 89.5) (width 1) (layer F.Cu) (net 17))
 (segment (start 137.5 89.5) (end 137.5 73) (width 1) (layer F.Cu) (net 17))
 (segment (start 137.5 73) (end 134 69.5) (width 1) (layer F.Cu) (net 17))
 (segment (start 134 69.5) (end 128.5 69.5) (width 1) (layer F.Cu) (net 17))
 (segment (start 128.5 69.5) (end 127 68) (width 1) (layer F.Cu) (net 17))
 (segment (start 127 68) (end 127 65) (width 1) (layer F.Cu) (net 17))
 (segment (start 127 65) (end 128 64) (width 1) (layer F.Cu) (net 17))
 (segment (start 128 64) (end 129.46 64) (width 1) (layer F.Cu) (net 17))
 (segment (start 129.46 64) (end 129.5 63.96) (width 1) (layer F.Cu) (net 17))
 (segment (start 164 64.04) (end 163.04 64.04) (width 1) (layer F.Cu) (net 16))
 (segment (start 163.04 64.04) (end 163 64) (width 1) (layer F.Cu) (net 16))
 (segment (start 163 64) (end 161.5 65.5) (width 1) (layer F.Cu) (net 16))
 (segment (start 161.5 65.5) (end 161.5 67) (width 1) (layer F.Cu) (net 16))
 (segment (start 161.5 67) (end 156 72.5) (width 1) (layer F.Cu) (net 16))
 (segment (start 156 72.5) (end 156 86.5) (width 1) (layer F.Cu) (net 16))
 (segment (start 156 86.5) (end 151 91.5) (width 1) (layer F.Cu) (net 16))
 (segment (start 151 91.5) (end 151 92) (width 1) (layer F.Cu) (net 16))
 (segment (start 164 77.54) (end 163.46 77.54) (width 1) (layer F.Cu) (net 13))
 (segment (start 163.46 77.54) (end 161.5 79.5) (width 1) (layer F.Cu) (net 13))
 (segment (start 161.5 79.5) (end 161.5 91.5) (width 1) (layer F.Cu) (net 13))
 (segment (start 161.5 91.5) (end 162 92) (width 1) (layer F.Cu) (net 13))
 (segment (start 135 74.5) (end 135 80.5) (width 0.75) (layer F.Cu) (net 11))
 (segment (start 135 80.5) (end 130 80.5) (width 0.75) (layer F.Cu) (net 11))
 (segment (start 130 80.5) (end 129.5 80) (width 0.75) (layer F.Cu) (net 11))
 (segment (start 135 67) (end 130 67) (width 0.75) (layer F.Cu) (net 15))
 (segment (start 130 67) (end 129.5 66.5) (width 0.75) (layer F.Cu) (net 15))
 (segment (start 135 61) (end 135 67) (width 0.75) (layer F.Cu) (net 15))
 (segment (start 164 75) (end 163.5 74.5) (width 0.75) (layer F.Cu) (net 14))
 (segment (start 163.5 74.5) (end 158.5 74.5) (width 0.75) (layer F.Cu) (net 14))
 (segment (start 158.5 74.5) (end 158.5 80.5) (width 0.75) (layer F.Cu) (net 14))
 (segment (start 158.5 61) (end 163.5 61) (width 0.75) (layer F.Cu) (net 12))
 (segment (start 163.5 61) (end 164 61.5) (width 0.75) (layer F.Cu) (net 12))
 (segment (start 158.5 61) (end 158.5 67) (width 0.75) (layer F.Cu) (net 12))
 (segment (start 136.88 54.62) (end 136.779 54.519) (width 0.25) (layer F.Cu) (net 6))
 (segment (start 136.779 54.519) (end 136.779 54.483) (width 0.25) (layer F.Cu) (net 6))
 (segment (start 136.88 54.62) (end 140 57.74) (width 0.75) (layer F.Cu) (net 6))
 (segment (start 140 57.74) (end 140 60) (width 0.75) (layer F.Cu) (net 6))
 (segment (start 140 60) (end 146 66) (width 0.75) (layer F.Cu) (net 6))
 (segment (start 146 66) (end 146 72.5) (width 0.75) (layer F.Cu) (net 6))
 (segment (start 146 72.5) (end 144 74.5) (width 0.75) (layer F.Cu) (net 6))
 (segment (start 141.96 56.79) (end 141.859 56.689) (width 0.25) (layer F.Cu) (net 2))
 (segment (start 141.859 56.689) (end 141.859 54.483) (width 0.25) (layer F.Cu) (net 2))
 (segment (start 141.96 56.79) (end 141.96 58.96) (width 0.75) (layer F.Cu) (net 2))
 (segment (start 141.96 58.96) (end 144 61) (width 0.75) (layer F.Cu) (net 2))
 (segment (start 141.96 54.62) (end 141.96 56.79) (width 0.75) (layer F.Cu) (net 2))
 (segment (start 157.658 55.422) (end 157.684 55.422) (width 0.25) (layer F.Cu) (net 8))
 (segment (start 157.684 55.422) (end 158.496 54.61) (width 0.25) (layer F.Cu) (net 8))
 (segment (start 157.658 55.422) (end 158.46 54.62) (width 0.75) (layer F.Cu) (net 8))
 (segment (start 149.5 74.5) (end 147.5 72.5) (width 0.75) (layer F.Cu) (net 8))
 (segment (start 147.5 72.5) (end 147.5 65.58) (width 0.75) (layer F.Cu) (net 8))
 (segment (start 147.5 65.58) (end 157.658 55.422) (width 0.75) (layer F.Cu) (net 8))
 (segment (start 153.416 54.61) (end 153.416 56.1351) (width 0.25) (layer F.Cu) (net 10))
 (segment (start 151.44 56.56) (end 152.9911 56.56) (width 0.25) (layer F.Cu) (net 10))
 (segment (start 152.9911 56.56) (end 153.416 56.1351) (width 0.25) (layer F.Cu) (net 10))
 (segment (start 151.44 56.56) (end 149.5 58.5) (width 0.75) (layer F.Cu) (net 10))
 (segment (start 149.5 58.5) (end 149.5 61) (width 0.75) (layer F.Cu) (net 10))
 (segment (start 153.38 54.62) (end 151.44 56.56) (width 0.75) (layer F.Cu) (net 10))
 (segment (start 141.0895 46.1295) (end 141.1255 46.1295) (width 0.25) (layer F.Cu) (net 5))
 (segment (start 141.1255 46.1295) (end 141.859 46.863) (width 0.25) (layer F.Cu) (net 5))
 (segment (start 141.0895 46.1295) (end 138.5 43.54) (width 0.5) (layer F.Cu) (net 5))
 (segment (start 138.5 43.54) (end 138.5 38) (width 0.5) (layer F.Cu) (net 5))
 (segment (start 141.96 47) (end 141.0895 46.1295) (width 0.5) (layer F.Cu) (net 5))
 (segment (start 136.44 46.56) (end 136.476 46.56) (width 0.25) (layer F.Cu) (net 1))
 (segment (start 136.476 46.56) (end 136.779 46.863) (width 0.25) (layer F.Cu) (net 1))
 (segment (start 136.44 46.56) (end 136 46.12) (width 0.5) (layer F.Cu) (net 1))
 (segment (start 136 46.12) (end 136 38) (width 0.5) (layer F.Cu) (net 1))
 (segment (start 136.88 47) (end 136.44 46.56) (width 0.5) (layer F.Cu) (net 1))
 (segment (start 158.46 46.23) (end 158.496 46.266) (width 0.25) (layer F.Cu) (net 9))
 (segment (start 158.496 46.266) (end 158.496 46.99) (width 0.25) (layer F.Cu) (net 9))
 (segment (start 158.46 46.23) (end 158.46 47) (width 0.5) (layer F.Cu) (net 9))
 (segment (start 153.21 40.2105) (end 158.46 45.46) (width 0.5) (layer F.Cu) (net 9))
 (segment (start 158.46 45.46) (end 158.46 46.23) (width 0.5) (layer F.Cu) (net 9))
 (segment (start 153.02 40.02) (end 153.21 40.2105) (width 0.5) (layer F.Cu) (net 9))
 (segment (start 152.5 38) (end 152.5 39.5) (width 0.5) (layer F.Cu) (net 9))
 (segment (start 152.5 39.5) (end 153.21 40.2105) (width 0.5) (layer F.Cu) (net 9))
 (segment (start 152.5 39.5) (end 153.02 40.02) (width 0.25) (layer F.Cu) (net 9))
 (segment (start 153.416 46.99) (end 153.416 45.4649) (width 0.25) (layer F.Cu) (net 7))
 (segment (start 151.69 45.31) (end 153.2611 45.31) (width 0.25) (layer F.Cu) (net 7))
 (segment (start 153.2611 45.31) (end 153.416 45.4649) (width 0.25) (layer F.Cu) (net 7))
 (segment (start 151.69 45.31) (end 150 43.62) (width 0.5) (layer F.Cu) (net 7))
 (segment (start 150 43.62) (end 150 38) (width 0.5) (layer F.Cu) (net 7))
 (segment (start 153.38 47) (end 151.69 45.31) (width 0.5) (layer F.Cu) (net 7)))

